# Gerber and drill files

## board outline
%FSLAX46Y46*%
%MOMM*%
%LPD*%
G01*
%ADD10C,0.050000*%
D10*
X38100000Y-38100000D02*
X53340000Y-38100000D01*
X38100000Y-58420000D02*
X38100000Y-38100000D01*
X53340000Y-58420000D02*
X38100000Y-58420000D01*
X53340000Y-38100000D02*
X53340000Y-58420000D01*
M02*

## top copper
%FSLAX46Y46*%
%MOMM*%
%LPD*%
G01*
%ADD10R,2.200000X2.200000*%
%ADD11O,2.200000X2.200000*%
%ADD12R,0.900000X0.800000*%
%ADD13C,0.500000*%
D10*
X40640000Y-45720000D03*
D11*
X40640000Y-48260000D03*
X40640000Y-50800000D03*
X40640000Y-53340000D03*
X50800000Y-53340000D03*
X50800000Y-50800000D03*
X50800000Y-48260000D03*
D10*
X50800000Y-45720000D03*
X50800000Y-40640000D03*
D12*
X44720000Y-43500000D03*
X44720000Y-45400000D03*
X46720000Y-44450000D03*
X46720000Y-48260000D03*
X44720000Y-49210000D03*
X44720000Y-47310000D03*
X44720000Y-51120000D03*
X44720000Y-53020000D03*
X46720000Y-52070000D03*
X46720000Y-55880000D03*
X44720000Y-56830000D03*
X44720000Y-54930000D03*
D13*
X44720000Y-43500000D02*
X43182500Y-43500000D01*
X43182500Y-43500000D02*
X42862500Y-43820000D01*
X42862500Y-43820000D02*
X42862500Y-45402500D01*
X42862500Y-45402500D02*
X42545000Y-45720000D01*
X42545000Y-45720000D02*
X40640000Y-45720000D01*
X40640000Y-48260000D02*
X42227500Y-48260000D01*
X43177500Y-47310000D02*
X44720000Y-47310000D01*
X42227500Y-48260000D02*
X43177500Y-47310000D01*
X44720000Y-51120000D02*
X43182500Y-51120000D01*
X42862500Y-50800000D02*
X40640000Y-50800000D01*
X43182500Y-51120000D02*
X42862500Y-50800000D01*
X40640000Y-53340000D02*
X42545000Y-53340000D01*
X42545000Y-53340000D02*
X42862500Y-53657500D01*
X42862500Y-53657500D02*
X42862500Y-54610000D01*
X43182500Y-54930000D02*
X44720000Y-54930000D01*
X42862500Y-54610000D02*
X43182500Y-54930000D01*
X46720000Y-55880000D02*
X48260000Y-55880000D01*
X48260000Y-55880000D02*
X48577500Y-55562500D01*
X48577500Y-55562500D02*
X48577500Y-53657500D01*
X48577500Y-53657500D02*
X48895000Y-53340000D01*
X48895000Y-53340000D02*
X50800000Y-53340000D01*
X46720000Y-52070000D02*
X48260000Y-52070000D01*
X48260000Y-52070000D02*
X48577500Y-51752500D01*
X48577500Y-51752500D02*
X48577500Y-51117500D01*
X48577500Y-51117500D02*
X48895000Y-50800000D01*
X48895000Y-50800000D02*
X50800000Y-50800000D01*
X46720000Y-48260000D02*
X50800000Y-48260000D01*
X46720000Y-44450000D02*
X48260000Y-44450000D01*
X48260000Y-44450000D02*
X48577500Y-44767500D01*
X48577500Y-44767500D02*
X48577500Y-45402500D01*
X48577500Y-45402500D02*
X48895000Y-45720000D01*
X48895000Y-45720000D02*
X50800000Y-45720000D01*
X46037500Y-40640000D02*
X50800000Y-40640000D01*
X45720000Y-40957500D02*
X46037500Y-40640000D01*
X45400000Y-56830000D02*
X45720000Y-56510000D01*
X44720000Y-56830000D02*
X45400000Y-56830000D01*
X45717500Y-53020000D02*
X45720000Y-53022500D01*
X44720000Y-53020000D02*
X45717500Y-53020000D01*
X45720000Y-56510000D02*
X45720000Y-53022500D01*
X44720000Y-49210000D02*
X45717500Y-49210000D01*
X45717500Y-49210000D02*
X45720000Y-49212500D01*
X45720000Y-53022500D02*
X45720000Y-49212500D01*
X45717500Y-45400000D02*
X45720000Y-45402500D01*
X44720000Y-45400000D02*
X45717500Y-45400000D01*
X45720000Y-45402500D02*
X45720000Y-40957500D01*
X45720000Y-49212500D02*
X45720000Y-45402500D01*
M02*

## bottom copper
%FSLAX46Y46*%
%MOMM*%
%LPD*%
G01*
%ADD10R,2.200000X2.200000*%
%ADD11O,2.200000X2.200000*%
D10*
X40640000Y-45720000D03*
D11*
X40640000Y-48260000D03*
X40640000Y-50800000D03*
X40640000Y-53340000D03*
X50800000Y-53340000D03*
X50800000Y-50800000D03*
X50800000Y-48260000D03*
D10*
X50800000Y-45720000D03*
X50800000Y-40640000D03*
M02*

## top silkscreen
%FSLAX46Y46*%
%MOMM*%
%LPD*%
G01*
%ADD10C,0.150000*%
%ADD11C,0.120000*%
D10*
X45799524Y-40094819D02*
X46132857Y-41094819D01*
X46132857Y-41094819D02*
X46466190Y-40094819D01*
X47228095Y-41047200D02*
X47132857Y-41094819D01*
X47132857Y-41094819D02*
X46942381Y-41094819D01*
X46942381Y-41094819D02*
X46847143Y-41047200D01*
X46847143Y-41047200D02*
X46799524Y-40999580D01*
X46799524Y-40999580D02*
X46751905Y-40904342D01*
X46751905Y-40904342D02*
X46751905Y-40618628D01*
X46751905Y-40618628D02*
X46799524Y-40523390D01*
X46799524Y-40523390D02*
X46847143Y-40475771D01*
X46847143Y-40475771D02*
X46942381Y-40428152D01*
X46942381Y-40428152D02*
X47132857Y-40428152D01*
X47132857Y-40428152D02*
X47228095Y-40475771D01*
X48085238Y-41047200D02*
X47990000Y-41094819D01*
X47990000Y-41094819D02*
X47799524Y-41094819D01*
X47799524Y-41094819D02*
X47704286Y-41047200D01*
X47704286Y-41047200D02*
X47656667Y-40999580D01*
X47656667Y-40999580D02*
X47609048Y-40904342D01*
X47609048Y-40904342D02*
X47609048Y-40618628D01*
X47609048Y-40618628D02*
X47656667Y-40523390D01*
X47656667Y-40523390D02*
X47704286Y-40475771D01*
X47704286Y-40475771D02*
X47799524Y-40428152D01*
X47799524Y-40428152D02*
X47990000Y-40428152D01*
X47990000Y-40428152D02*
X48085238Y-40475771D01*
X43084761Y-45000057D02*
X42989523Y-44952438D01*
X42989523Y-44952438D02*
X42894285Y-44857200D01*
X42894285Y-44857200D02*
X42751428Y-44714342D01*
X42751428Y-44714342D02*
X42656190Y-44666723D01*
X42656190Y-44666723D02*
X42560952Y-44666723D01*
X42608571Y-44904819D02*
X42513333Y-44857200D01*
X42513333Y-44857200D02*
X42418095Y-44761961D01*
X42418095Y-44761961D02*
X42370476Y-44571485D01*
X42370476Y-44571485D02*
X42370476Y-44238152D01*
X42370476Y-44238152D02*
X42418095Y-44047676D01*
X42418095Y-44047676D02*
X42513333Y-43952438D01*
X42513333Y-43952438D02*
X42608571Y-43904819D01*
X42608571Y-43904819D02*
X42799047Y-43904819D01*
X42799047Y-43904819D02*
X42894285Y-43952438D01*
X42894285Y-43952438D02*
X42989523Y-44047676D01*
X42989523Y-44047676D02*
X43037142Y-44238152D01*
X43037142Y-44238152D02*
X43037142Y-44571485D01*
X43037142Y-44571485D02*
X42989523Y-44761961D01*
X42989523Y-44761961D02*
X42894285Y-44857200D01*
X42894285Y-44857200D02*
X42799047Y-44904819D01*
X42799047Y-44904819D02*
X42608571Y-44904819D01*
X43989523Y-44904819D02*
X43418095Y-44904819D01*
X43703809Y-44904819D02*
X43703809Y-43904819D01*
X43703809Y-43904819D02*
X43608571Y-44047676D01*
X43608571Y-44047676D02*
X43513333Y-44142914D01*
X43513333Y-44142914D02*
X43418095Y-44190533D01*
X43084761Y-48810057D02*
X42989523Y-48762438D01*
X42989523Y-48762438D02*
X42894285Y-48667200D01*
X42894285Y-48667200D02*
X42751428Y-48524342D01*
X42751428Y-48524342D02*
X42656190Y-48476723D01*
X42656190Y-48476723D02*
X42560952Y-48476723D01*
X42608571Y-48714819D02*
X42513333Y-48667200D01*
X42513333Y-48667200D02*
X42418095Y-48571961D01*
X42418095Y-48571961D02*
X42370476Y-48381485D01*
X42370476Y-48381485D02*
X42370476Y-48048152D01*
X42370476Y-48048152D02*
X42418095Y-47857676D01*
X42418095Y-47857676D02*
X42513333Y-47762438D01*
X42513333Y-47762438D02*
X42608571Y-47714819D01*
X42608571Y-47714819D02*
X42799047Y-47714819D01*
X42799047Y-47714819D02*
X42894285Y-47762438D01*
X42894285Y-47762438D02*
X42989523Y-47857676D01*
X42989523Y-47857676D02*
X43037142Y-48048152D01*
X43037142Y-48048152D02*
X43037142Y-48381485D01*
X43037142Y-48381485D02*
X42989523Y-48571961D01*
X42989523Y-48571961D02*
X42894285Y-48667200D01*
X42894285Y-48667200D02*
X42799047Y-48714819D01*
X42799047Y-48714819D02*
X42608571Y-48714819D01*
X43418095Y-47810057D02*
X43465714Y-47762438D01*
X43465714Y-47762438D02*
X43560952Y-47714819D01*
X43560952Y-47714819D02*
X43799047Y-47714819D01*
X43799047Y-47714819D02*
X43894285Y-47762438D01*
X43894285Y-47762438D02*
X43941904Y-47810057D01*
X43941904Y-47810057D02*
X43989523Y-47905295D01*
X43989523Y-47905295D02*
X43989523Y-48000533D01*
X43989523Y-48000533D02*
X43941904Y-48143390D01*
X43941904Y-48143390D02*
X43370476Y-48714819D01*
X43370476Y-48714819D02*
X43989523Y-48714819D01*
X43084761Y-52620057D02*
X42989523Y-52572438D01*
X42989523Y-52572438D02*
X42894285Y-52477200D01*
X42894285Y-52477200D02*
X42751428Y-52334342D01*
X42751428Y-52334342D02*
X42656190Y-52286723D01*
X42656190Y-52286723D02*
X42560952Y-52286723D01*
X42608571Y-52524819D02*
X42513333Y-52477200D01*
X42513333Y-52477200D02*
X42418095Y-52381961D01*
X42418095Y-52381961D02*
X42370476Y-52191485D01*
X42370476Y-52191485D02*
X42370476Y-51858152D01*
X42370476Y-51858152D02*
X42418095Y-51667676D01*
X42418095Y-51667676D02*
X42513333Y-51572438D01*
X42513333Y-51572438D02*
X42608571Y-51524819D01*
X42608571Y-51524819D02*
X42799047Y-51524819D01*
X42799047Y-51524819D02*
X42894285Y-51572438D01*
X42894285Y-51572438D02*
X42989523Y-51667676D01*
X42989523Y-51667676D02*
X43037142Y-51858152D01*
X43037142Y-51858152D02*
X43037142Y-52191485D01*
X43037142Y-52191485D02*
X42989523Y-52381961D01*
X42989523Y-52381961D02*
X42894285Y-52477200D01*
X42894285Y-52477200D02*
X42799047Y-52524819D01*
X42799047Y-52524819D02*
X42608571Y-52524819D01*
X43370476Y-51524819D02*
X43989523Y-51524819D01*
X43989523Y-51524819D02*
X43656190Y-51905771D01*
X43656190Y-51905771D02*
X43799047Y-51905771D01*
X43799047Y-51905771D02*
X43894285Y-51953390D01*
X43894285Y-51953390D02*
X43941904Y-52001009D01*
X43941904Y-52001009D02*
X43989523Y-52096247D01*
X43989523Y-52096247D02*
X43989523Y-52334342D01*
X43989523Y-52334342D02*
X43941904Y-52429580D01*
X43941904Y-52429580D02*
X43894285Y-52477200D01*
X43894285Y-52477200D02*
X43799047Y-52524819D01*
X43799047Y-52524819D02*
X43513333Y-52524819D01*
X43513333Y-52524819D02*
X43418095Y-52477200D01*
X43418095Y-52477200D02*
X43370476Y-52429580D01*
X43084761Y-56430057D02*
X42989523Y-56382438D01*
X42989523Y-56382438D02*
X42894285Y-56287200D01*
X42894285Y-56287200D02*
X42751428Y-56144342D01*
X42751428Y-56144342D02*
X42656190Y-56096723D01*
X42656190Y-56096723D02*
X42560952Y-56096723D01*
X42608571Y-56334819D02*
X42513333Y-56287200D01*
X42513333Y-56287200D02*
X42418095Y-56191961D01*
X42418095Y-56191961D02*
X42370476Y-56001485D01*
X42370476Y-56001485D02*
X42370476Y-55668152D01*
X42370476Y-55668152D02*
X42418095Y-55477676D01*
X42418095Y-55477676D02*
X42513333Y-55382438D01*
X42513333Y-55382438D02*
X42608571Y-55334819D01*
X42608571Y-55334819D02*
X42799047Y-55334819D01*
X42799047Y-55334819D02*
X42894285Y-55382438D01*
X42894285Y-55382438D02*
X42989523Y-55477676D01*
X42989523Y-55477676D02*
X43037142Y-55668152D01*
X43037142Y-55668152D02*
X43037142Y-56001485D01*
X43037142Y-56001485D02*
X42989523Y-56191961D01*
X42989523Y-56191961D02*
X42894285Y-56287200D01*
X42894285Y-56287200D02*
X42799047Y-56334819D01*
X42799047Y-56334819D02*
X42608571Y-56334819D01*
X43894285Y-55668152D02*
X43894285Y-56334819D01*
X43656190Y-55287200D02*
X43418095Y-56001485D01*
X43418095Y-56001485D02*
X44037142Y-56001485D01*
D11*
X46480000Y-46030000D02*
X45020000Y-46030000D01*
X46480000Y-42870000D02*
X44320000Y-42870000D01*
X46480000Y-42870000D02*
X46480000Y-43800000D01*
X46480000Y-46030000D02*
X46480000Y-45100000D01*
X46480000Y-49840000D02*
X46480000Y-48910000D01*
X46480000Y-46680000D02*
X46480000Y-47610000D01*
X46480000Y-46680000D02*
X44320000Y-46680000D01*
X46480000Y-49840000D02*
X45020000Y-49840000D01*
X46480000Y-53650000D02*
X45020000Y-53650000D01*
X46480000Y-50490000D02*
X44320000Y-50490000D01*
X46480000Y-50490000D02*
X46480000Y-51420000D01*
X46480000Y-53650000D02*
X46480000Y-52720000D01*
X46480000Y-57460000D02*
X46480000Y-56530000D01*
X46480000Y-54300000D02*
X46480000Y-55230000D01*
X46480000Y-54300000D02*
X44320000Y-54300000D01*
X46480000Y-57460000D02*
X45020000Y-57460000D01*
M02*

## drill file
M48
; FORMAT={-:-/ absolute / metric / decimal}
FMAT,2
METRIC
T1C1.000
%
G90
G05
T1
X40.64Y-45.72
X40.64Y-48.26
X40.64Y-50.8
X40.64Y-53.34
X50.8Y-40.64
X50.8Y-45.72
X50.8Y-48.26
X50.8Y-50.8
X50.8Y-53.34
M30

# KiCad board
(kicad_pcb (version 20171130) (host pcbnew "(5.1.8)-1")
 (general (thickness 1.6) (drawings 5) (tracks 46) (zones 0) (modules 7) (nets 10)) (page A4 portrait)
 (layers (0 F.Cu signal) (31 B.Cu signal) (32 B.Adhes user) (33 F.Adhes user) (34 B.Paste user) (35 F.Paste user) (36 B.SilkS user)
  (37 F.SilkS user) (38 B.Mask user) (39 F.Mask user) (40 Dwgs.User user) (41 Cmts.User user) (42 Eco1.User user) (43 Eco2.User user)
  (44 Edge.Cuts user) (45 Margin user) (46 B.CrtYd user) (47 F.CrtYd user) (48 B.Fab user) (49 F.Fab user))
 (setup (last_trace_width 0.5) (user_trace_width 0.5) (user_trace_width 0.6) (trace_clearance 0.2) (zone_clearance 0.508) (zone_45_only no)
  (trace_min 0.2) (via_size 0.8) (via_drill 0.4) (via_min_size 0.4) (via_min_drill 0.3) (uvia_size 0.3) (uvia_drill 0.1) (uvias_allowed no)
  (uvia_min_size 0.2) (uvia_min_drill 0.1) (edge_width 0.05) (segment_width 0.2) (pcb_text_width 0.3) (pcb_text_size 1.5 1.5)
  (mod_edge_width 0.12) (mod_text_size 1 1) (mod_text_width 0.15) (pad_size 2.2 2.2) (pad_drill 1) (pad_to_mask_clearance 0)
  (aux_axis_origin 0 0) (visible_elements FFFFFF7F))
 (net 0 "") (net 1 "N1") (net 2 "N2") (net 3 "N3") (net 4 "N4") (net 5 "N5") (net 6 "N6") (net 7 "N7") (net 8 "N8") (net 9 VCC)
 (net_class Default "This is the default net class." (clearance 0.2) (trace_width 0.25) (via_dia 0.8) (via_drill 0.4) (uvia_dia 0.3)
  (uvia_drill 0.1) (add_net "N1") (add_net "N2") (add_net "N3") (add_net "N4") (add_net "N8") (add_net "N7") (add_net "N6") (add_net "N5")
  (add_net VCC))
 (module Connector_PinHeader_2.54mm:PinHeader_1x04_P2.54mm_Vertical (layer B.Cu) (at 40.64 45.72 180)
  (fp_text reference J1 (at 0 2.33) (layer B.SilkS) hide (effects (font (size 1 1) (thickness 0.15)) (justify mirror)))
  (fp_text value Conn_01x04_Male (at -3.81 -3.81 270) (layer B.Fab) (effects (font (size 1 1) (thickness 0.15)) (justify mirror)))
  (pad 1 thru_hole rect (at 0 0 180) (size 2.2 2.2) (drill 1) (layers *.Cu *.Mask) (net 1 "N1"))
  (pad 2 thru_hole oval (at 0 -2.54 180) (size 2.2 2.2) (drill 1) (layers *.Cu *.Mask) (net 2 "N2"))
  (pad 3 thru_hole oval (at 0 -5.08 180) (size 2.2 2.2) (drill 1) (layers *.Cu *.Mask) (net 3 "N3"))
  (pad 4 thru_hole oval (at 0 -7.62 180) (size 2.2 2.2) (drill 1) (layers *.Cu *.Mask) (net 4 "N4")))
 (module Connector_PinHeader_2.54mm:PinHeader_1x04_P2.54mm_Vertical (layer B.Cu) (at 50.8 45.72 180)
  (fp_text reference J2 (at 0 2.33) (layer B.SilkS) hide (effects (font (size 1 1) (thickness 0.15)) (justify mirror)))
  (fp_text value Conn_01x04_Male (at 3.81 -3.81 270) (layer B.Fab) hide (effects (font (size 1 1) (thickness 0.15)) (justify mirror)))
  (pad 4 thru_hole oval (at 0 -7.62 180) (size 2.2 2.2) (drill 1) (layers *.Cu *.Mask) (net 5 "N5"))
  (pad 3 thru_hole oval (at 0 -5.08 180) (size 2.2 2.2) (drill 1) (layers *.Cu *.Mask) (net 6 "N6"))
  (pad 2 thru_hole oval (at 0 -2.54 180) (size 2.2 2.2) (drill 1) (layers *.Cu *.Mask) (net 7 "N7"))
  (pad 1 thru_hole rect (at 0 0 180) (size 2.2 2.2) (drill 1) (layers *.Cu *.Mask) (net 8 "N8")))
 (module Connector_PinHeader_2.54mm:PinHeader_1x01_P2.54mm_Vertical (layer B.Cu) (at 50.8 40.64)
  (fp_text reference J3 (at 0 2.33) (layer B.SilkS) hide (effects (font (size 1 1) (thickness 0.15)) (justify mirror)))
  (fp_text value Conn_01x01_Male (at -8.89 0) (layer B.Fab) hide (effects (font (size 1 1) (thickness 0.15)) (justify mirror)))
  (pad 1 thru_hole rect (at 0 0) (size 2.2 2.2) (drill 1) (layers *.Cu *.Mask) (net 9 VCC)))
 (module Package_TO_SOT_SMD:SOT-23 (layer F.Cu) (at 45.72 44.45)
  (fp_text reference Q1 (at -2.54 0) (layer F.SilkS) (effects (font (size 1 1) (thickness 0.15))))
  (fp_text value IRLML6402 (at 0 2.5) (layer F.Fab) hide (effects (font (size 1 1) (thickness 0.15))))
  (fp_line (start 0.76 1.58) (end -0.7 1.58) (layer F.SilkS) (width 0.12))
  (fp_line (start 0.76 -1.58) (end -1.4 -1.58) (layer F.SilkS) (width 0.12))
  (fp_line (start 0.76 -1.58) (end 0.76 -0.65) (layer F.SilkS) (width 0.12))
  (fp_line (start 0.76 1.58) (end 0.76 0.65) (layer F.SilkS) (width 0.12))
  (pad 1 smd rect (at -1 -0.95) (size 0.9 0.8) (layers F.Cu F.Paste F.Mask) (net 1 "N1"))
  (pad 2 smd rect (at -1 0.95) (size 0.9 0.8) (layers F.Cu F.Paste F.Mask) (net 9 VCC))
  (pad 3 smd rect (at 1 0) (size 0.9 0.8) (layers F.Cu F.Paste F.Mask) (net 8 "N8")))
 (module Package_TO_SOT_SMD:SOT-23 (layer F.Cu) (at 45.72 48.26)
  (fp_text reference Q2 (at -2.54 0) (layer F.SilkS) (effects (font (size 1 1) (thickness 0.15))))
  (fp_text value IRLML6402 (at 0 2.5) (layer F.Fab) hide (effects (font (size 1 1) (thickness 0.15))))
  (fp_line (start 0.76 1.58) (end 0.76 0.65) (layer F.SilkS) (width 0.12))
  (fp_line (start 0.76 -1.58) (end 0.76 -0.65) (layer F.SilkS) (width 0.12))
  (fp_line (start 0.76 -1.58) (end -1.4 -1.58) (layer F.SilkS) (width 0.12))
  (fp_line (start 0.76 1.58) (end -0.7 1.58) (layer F.SilkS) (width 0.12))
  (pad 3 smd rect (at 1 0) (size 0.9 0.8) (layers F.Cu F.Paste F.Mask) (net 7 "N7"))
  (pad 2 smd rect (at -1 0.95) (size 0.9 0.8) (layers F.Cu F.Paste F.Mask) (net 9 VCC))
  (pad 1 smd rect (at -1 -0.95) (size 0.9 0.8) (layers F.Cu F.Paste F.Mask) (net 2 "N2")))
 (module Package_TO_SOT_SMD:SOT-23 (layer F.Cu) (at 45.72 52.07)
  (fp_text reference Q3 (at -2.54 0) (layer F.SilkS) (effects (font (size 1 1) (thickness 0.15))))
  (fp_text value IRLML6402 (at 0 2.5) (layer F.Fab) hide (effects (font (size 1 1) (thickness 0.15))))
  (fp_line (start 0.76 1.58) (end -0.7 1.58) (layer F.SilkS) (width 0.12))
  (fp_line (start 0.76 -1.58) (end -1.4 -1.58) (layer F.SilkS) (width 0.12))
  (fp_line (start 0.76 -1.58) (end 0.76 -0.65) (layer F.SilkS) (width 0.12))
  (fp_line (start 0.76 1.58) (end 0.76 0.65) (layer F.SilkS) (width 0.12))
  (pad 1 smd rect (at -1 -0.95) (size 0.9 0.8) (layers F.Cu F.Paste F.Mask) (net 3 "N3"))
  (pad 2 smd rect (at -1 0.95) (size 0.9 0.8) (layers F.Cu F.Paste F.Mask) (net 9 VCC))
  (pad 3 smd rect (at 1 0) (size 0.9 0.8) (layers F.Cu F.Paste F.Mask) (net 6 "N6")))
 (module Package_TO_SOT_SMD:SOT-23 (layer F.Cu) (at 45.72 55.88)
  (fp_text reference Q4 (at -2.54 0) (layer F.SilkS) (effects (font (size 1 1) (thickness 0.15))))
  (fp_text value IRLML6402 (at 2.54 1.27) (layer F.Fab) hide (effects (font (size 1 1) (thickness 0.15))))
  (fp_line (start 0.76 1.58) (end 0.76 0.65) (layer F.SilkS) (width 0.12))
  (fp_line (start 0.76 -1.58) (end 0.76 -0.65) (layer F.SilkS) (width 0.12))
  (fp_line (start 0.76 -1.58) (end -1.4 -1.58) (layer F.SilkS) (width 0.12))
  (fp_line (start 0.76 1.58) (end -0.7 1.58) (layer F.SilkS) (width 0.12))
  (pad 3 smd rect (at 1 0) (size 0.9 0.8) (layers F.Cu F.Paste F.Mask) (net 5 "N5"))
  (pad 2 smd rect (at -1 0.95) (size 0.9 0.8) (layers F.Cu F.Paste F.Mask) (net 9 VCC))
  (pad 1 smd rect (at -1 -0.95) (size 0.9 0.8) (layers F.Cu F.Paste F.Mask) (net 4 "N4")))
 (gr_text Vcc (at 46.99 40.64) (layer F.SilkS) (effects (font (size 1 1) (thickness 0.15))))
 (gr_line (start 38.1 38.1) (end 53.34 38.1) (layer Edge.Cuts) (width 0.05))
 (gr_line (start 38.1 58.42) (end 38.1 38.1) (layer Edge.Cuts) (width 0.05))
 (gr_line (start 53.34 58.42) (end 38.1 58.42) (layer Edge.Cuts) (width 0.05))
 (gr_line (start 53.34 38.1) (end 53.34 58.42) (layer Edge.Cuts) (width 0.05))
 (segment (start 44.72 43.5) (end 43.1825 43.5) (width 0.5) (layer F.Cu) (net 1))
 (segment (start 43.1825 43.5) (end 42.8625 43.82) (width 0.5) (layer F.Cu) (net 1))
 (segment (start 42.8625 43.82) (end 42.8625 45.4025) (width 0.5) (layer F.Cu) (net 1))
 (segment (start 42.8625 45.4025) (end 42.545 45.72) (width 0.5) (layer F.Cu) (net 1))
 (segment (start 42.545 45.72) (end 40.64 45.72) (width 0.5) (layer F.Cu) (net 1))
 (segment (start 40.64 48.26) (end 42.2275 48.26) (width 0.5) (layer F.Cu) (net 2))
 (segment (start 43.1775 47.31) (end 44.72 47.31) (width 0.5) (layer F.Cu) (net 2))
 (segment (start 42.2275 48.26) (end 43.1775 47.31) (width 0.5) (layer F.Cu) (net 2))
 (segment (start 44.72 51.12) (end 43.1825 51.12) (width 0.5) (layer F.Cu) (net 3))
 (segment (start 42.8625 50.8) (end 40.64 50.8) (width 0.5) (layer F.Cu) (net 3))
 (segment (start 43.1825 51.12) (end 42.8625 50.8) (width 0.5) (layer F.Cu) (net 3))
 (segment (start 40.64 53.34) (end 42.545 53.34) (width 0.5) (layer F.Cu) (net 4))
 (segment (start 42.545 53.34) (end 42.8625 53.6575) (width 0.5) (layer F.Cu) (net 4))
 (segment (start 42.8625 53.6575) (end 42.8625 54.61) (width 0.5) (layer F.Cu) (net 4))
 (segment (start 43.1825 54.93) (end 44.72 54.93) (width 0.5) (layer F.Cu) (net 4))
 (segment (start 42.8625 54.61) (end 43.1825 54.93) (width 0.5) (layer F.Cu) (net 4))
 (segment (start 46.72 55.88) (end 48.26 55.88) (width 0.5) (layer F.Cu) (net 5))
 (segment (start 48.26 55.88) (end 48.5775 55.5625) (width 0.5) (layer F.Cu) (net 5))
 (segment (start 48.5775 55.5625) (end 48.5775 53.6575) (width 0.5) (layer F.Cu) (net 5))
 (segment (start 48.5775 53.6575) (end 48.895 53.34) (width 0.5) (layer F.Cu) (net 5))
 (segment (start 48.895 53.34) (end 50.8 53.34) (width 0.5) (layer F.Cu) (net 5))
 (segment (start 46.72 52.07) (end 48.26 52.07) (width 0.5) (layer F.Cu) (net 6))
 (segment (start 48.26 52.07) (end 48.5775 51.7525) (width 0.5) (layer F.Cu) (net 6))
 (segment (start 48.5775 51.7525) (end 48.5775 51.1175) (width 0.5) (layer F.Cu) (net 6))
 (segment (start 48.5775 51.1175) (end 48.895 50.8) (width 0.5) (layer F.Cu) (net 6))
 (segment (start 48.895 50.8) (end 50.8 50.8) (width 0.5) (layer F.Cu) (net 6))
 (segment (start 46.72 48.26) (end 50.8 48.26) (width 0.5) (layer F.Cu) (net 7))
 (segment (start 46.72 44.45) (end 48.26 44.45) (width 0.5) (layer F.Cu) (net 8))
 (segment (start 48.26 44.45) (end 48.5775 44.7675) (width 0.5) (layer F.Cu) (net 8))
 (segment (start 48.5775 44.7675) (end 48.5775 45.4025) (width 0.5) (layer F.Cu) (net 8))
 (segment (start 48.5775 45.4025) (end 48.895 45.72) (width 0.5) (layer F.Cu) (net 8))
 (segment (start 48.895 45.72) (end 50.8 45.72) (width 0.5) (layer F.Cu) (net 8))
 (segment (start 46.0375 40.64) (end 50.8 40.64) (width 0.5) (layer F.Cu) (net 9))
 (segment (start 45.72 40.9575) (end 46.0375 40.64) (width 0.5) (layer F.Cu) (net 9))
 (segment (start 45.4 56.83) (end 45.72 56.51) (width 0.5) (layer F.Cu) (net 9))
 (segment (start 44.72 56.83) (end 45.4 56.83) (width 0.5) (layer F.Cu) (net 9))
 (segment (start 45.7175 53.02) (end 45.72 53.0225) (width 0.5) (layer F.Cu) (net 9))
 (segment (start 44.72 53.02) (end 45.7175 53.02) (width 0.5) (layer F.Cu) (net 9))
 (segment (start 45.72 56.51) (end 45.72 53.0225) (width 0.5) (layer F.Cu) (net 9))
 (segment (start 44.72 49.21) (end 45.7175 49.21) (width 0.5) (layer F.Cu) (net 9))
 (segment (start 45.7175 49.21) (end 45.72 49.2125) (width 0.5) (layer F.Cu) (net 9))
 (segment (start 45.72 53.0225) (end 45.72 49.2125) (width 0.5) (layer F.Cu) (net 9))
 (segment (start 45.7175 45.4) (end 45.72 45.4025) (width 0.5) (layer F.Cu) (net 9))
 (segment (start 44.72 45.4) (end 45.7175 45.4) (width 0.5) (layer F.Cu) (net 9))
 (segment (start 45.72 45.4025) (end 45.72 40.9575) (width 0.5) (layer F.Cu) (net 9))
 (segment (start 45.72 49.2125) (end 45.72 45.4025) (width 0.5) (layer F.Cu) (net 9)))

